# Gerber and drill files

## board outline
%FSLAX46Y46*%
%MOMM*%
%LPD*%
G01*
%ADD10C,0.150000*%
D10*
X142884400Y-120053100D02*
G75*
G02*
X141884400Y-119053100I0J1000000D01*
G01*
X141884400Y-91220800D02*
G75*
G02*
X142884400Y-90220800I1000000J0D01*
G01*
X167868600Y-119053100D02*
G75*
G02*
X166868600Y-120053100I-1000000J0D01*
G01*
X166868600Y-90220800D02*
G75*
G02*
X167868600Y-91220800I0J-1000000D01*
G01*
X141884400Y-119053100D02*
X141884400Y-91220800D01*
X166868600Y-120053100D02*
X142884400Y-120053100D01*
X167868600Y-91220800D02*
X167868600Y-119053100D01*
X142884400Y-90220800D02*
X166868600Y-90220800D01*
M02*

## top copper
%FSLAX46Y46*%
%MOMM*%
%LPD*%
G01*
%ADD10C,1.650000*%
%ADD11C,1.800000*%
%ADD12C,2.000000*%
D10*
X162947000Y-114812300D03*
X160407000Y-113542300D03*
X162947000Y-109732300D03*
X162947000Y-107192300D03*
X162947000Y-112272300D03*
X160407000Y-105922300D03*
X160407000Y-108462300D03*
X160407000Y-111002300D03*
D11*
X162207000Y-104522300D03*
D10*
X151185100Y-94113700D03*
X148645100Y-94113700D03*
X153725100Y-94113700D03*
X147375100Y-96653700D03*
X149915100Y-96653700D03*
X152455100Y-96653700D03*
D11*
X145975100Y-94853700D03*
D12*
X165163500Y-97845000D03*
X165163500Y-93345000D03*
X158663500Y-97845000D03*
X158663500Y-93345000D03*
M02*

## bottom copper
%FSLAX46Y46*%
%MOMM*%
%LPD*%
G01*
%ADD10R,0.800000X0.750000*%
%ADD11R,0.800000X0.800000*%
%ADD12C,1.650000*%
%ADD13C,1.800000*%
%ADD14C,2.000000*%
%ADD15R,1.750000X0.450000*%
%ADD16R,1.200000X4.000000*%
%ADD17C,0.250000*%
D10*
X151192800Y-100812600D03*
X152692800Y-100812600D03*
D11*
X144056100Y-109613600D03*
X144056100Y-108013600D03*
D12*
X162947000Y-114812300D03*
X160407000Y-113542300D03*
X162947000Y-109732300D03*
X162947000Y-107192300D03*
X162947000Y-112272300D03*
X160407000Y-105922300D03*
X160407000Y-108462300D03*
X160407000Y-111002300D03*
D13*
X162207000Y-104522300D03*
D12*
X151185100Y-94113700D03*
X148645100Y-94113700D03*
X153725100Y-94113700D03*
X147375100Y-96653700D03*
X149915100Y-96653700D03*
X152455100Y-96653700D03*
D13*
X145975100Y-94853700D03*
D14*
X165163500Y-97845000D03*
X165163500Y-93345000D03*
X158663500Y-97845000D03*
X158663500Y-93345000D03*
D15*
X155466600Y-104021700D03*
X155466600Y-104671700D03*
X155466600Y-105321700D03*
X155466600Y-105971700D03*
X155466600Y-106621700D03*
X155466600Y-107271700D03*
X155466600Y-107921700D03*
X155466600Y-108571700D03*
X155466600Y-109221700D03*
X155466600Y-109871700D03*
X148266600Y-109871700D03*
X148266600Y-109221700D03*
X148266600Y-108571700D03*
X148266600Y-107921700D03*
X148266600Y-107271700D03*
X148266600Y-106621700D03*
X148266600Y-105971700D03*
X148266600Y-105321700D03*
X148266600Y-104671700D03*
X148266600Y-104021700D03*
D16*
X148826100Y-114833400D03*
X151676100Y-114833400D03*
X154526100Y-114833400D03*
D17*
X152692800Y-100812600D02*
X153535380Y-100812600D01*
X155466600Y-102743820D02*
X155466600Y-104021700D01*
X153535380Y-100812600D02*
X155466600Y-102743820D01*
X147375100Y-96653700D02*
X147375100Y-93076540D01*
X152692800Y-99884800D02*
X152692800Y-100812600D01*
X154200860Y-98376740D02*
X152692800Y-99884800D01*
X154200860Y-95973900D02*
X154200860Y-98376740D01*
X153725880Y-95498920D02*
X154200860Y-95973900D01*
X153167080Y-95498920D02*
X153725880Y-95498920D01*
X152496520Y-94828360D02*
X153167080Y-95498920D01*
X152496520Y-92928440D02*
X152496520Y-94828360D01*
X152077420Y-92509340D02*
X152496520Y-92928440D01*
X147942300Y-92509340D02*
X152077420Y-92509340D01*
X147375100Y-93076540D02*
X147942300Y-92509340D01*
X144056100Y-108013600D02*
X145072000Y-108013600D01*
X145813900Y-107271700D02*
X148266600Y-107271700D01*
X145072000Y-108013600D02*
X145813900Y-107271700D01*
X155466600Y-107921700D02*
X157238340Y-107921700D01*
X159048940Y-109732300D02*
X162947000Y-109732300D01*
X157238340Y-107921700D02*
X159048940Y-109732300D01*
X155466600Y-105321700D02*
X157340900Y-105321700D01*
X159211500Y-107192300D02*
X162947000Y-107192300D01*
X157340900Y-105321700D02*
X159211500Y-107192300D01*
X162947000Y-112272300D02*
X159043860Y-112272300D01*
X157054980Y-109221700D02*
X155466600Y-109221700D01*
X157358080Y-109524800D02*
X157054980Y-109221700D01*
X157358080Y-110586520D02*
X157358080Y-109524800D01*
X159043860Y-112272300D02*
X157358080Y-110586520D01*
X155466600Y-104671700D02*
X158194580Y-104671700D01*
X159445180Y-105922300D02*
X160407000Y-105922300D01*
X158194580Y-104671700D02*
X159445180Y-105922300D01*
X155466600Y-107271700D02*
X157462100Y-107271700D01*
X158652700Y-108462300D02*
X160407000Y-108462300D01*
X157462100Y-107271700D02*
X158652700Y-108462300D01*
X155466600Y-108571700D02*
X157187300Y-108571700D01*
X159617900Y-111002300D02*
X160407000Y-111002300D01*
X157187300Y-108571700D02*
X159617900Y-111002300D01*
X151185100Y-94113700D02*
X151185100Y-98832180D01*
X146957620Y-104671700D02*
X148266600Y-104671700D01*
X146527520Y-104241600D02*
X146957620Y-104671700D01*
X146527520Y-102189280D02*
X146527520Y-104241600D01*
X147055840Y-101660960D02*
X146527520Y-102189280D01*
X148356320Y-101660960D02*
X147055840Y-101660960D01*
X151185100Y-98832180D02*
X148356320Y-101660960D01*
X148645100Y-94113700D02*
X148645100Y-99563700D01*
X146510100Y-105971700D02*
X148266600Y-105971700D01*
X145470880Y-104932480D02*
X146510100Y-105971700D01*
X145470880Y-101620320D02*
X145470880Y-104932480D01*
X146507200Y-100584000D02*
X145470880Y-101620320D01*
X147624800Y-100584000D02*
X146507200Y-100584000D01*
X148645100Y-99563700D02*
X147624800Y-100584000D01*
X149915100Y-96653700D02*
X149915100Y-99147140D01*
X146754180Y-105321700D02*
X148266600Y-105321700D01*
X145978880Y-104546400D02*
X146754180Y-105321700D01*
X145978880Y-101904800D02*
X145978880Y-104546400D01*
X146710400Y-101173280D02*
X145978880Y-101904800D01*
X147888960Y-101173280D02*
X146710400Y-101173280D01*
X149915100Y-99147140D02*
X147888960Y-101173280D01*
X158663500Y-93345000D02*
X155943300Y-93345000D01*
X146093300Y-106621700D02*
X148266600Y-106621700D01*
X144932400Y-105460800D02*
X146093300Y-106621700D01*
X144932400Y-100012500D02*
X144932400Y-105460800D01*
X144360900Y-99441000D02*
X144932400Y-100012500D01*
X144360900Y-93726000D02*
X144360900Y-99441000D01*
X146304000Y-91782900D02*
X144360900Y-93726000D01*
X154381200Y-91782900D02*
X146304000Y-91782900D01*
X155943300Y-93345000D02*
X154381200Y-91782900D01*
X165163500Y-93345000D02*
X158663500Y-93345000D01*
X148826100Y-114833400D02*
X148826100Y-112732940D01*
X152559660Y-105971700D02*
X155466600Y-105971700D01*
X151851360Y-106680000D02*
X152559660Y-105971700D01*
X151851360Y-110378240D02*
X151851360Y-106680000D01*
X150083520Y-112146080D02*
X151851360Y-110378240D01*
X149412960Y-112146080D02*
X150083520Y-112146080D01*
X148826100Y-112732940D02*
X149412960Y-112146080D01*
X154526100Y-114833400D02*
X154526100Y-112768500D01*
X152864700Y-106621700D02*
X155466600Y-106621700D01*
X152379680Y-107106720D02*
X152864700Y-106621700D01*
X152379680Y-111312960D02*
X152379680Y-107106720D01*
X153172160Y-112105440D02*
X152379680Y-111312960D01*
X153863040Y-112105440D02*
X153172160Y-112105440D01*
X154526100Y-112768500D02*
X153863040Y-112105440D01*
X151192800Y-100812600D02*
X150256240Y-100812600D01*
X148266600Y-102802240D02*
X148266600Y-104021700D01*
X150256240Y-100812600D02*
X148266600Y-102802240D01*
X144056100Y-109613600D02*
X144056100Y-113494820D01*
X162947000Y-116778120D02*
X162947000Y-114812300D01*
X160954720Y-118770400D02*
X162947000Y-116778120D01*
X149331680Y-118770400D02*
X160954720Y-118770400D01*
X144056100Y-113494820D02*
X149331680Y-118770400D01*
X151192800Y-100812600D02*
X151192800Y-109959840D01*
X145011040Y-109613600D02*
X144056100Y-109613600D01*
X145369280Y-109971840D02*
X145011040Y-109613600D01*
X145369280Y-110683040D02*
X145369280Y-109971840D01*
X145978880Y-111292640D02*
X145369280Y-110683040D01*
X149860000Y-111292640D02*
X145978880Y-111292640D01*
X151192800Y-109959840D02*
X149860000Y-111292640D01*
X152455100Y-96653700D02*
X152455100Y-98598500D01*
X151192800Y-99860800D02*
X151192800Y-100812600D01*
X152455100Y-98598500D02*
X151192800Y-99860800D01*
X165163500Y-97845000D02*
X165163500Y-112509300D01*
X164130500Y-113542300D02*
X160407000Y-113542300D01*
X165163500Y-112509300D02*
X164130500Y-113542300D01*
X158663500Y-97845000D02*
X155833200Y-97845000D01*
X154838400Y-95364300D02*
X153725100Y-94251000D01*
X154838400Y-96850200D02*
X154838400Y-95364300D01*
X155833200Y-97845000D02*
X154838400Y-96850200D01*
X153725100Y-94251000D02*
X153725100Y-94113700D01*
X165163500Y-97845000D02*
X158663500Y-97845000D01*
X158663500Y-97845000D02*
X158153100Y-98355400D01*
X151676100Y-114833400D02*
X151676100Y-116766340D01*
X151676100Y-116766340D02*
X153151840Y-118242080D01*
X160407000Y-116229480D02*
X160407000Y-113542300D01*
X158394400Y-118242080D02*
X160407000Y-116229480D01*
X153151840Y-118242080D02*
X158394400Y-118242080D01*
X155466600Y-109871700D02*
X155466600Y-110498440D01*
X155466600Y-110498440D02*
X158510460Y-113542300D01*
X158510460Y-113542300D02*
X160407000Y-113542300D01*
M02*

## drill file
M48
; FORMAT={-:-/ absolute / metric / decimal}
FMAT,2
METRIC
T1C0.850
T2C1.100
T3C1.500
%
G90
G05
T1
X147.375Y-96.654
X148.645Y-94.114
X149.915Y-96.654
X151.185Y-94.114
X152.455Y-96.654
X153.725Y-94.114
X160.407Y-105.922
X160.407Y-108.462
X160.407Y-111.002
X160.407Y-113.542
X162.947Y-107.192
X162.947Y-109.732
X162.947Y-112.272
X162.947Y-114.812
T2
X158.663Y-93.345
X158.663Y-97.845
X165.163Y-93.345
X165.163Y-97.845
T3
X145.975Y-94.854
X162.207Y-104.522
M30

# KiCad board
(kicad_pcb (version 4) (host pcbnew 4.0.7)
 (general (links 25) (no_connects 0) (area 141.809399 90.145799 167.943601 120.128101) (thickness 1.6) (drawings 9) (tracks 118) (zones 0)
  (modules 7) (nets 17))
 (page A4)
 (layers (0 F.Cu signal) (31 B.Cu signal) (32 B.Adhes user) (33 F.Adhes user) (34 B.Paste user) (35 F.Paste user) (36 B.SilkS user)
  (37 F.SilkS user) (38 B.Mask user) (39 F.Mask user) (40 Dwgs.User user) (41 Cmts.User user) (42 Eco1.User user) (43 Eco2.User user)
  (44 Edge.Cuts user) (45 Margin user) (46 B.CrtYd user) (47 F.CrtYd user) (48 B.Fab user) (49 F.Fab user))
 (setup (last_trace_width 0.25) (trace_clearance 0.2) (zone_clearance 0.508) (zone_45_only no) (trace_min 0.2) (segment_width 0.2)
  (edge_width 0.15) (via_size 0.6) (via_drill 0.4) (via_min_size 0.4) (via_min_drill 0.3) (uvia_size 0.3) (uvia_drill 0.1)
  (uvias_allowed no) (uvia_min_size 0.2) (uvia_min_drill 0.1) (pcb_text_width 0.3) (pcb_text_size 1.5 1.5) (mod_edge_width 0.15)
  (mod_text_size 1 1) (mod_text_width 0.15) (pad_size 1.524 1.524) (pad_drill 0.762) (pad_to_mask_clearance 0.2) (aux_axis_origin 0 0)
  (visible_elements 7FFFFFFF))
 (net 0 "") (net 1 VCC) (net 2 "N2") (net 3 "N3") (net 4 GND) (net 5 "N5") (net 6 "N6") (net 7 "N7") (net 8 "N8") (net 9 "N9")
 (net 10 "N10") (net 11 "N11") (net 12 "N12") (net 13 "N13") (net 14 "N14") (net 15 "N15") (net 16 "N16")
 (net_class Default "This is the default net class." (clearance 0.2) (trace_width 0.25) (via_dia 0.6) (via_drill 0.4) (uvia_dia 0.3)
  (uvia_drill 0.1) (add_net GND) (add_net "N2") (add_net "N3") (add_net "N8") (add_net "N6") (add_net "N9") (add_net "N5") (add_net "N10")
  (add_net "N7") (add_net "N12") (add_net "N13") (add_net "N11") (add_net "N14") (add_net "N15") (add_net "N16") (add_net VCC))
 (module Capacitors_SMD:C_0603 (layer B.Cu) (at 151.9428 100.8126 180)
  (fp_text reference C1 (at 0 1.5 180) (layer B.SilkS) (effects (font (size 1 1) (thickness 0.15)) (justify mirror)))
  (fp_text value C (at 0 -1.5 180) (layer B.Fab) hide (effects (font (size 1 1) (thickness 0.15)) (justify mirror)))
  (pad 2 smd rect (at 0.75 0 180) (size 0.8 0.75) (layers B.Cu B.Paste B.Mask) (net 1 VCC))
  (pad 1 smd rect (at -0.75 0 180) (size 0.8 0.75) (layers B.Cu B.Paste B.Mask) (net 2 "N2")))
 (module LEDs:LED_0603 (layer B.Cu) (at 144.0561 108.8136 270)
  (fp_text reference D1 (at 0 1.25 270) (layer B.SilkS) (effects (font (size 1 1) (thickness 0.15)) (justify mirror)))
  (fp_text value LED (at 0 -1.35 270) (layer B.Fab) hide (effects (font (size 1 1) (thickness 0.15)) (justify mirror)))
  (pad 2 smd rect (at 0.8 0 90) (size 0.8 0.8) (layers B.Cu B.Paste B.Mask) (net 1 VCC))
  (pad 1 smd rect (at -0.8 0 90) (size 0.8 0.8) (layers B.Cu B.Paste B.Mask) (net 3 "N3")))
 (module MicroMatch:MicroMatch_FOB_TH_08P (layer F.Cu) (at 166.497 106.0323 90)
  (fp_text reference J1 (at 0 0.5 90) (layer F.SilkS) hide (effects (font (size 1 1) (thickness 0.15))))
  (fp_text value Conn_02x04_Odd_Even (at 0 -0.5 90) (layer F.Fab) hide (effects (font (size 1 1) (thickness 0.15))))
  (pad 8 thru_hole circle (at -8.78 -3.55 90) (size 1.65 1.65) (drill 0.85) (layers *.Cu *.Mask) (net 1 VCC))
  (pad 7 thru_hole circle (at -7.51 -6.09 90) (size 1.65 1.65) (drill 0.85) (layers *.Cu *.Mask) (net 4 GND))
  (pad 4 thru_hole circle (at -3.7 -3.55 90) (size 1.65 1.65) (drill 0.85) (layers *.Cu *.Mask) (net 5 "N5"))
  (pad 2 thru_hole circle (at -1.16 -3.55 90) (size 1.65 1.65) (drill 0.85) (layers *.Cu *.Mask) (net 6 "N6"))
  (pad 6 thru_hole circle (at -6.24 -3.55 90) (size 1.65 1.65) (drill 0.85) (layers *.Cu *.Mask) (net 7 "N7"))
  (pad 1 thru_hole circle (at 0.11 -6.09 90) (size 1.65 1.65) (drill 0.85) (layers *.Cu *.Mask) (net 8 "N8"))
  (pad 3 thru_hole circle (at -2.43 -6.09 90) (size 1.65 1.65) (drill 0.85) (layers *.Cu *.Mask) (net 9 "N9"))
  (pad 5 thru_hole circle (at -4.97 -6.09 90) (size 1.65 1.65) (drill 0.85) (layers *.Cu *.Mask) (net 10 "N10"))
  (pad "" np_thru_hole circle (at 1.51 -4.29 90) (size 1.8 1.8) (drill 1.5) (layers *.Cu *.Mask)))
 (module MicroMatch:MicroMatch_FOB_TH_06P (layer F.Cu) (at 147.4851 90.5637 180)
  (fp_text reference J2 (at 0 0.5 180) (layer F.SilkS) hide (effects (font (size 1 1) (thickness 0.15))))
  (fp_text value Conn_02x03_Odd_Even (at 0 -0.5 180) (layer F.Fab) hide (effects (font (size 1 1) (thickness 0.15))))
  (pad 4 thru_hole circle (at -3.7 -3.55 180) (size 1.65 1.65) (drill 0.85) (layers *.Cu *.Mask) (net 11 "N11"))
  (pad 2 thru_hole circle (at -1.16 -3.55 180) (size 1.65 1.65) (drill 0.85) (layers *.Cu *.Mask) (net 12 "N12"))
  (pad 6 thru_hole circle (at -6.24 -3.55 180) (size 1.65 1.65) (drill 0.85) (layers *.Cu *.Mask) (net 4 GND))
  (pad 1 thru_hole circle (at 0.11 -6.09 180) (size 1.65 1.65) (drill 0.85) (layers *.Cu *.Mask) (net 2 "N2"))
  (pad 3 thru_hole circle (at -2.43 -6.09 180) (size 1.65 1.65) (drill 0.85) (layers *.Cu *.Mask) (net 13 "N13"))
  (pad 5 thru_hole circle (at -4.97 -6.09 180) (size 1.65 1.65) (drill 0.85) (layers *.Cu *.Mask) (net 1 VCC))
  (pad "" np_thru_hole circle (at 1.51 -4.29 180) (size 1.8 1.8) (drill 1.5) (layers *.Cu *.Mask)))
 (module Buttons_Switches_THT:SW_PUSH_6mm (layer B.Cu) (at 165.1635 93.345 180)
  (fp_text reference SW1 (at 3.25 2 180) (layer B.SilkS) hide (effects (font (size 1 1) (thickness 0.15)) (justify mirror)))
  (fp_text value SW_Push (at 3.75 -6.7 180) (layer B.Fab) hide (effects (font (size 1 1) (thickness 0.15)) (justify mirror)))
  (pad 2 thru_hole circle (at 0 -4.5 90) (size 2 2) (drill 1.1) (layers *.Cu *.Mask) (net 4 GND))
  (pad 1 thru_hole circle (at 0 0 90) (size 2 2) (drill 1.1) (layers *.Cu *.Mask) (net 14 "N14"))
  (pad 2 thru_hole circle (at 6.5 -4.5 90) (size 2 2) (drill 1.1) (layers *.Cu *.Mask) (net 4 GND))
  (pad 1 thru_hole circle (at 6.5 0 90) (size 2 2) (drill 1.1) (layers *.Cu *.Mask) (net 14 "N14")))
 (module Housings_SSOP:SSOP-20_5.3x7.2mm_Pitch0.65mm (layer B.Cu) (at 151.8666 106.9467 180)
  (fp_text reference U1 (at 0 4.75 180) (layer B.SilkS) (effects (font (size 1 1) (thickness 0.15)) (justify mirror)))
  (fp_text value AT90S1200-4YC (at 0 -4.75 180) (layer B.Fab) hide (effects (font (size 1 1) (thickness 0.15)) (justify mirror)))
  (pad 1 smd rect (at -3.6 2.925 180) (size 1.75 0.45) (layers B.Cu B.Paste B.Mask) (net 2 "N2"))
  (pad 2 smd rect (at -3.6 2.275 180) (size 1.75 0.45) (layers B.Cu B.Paste B.Mask) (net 8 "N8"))
  (pad 3 smd rect (at -3.6 1.625 180) (size 1.75 0.45) (layers B.Cu B.Paste B.Mask) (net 6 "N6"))
  (pad 4 smd rect (at -3.6 0.975 180) (size 1.75 0.45) (layers B.Cu B.Paste B.Mask) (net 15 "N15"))
  (pad 5 smd rect (at -3.6 0.325 180) (size 1.75 0.45) (layers B.Cu B.Paste B.Mask) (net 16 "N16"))
  (pad 6 smd rect (at -3.6 -0.325 180) (size 1.75 0.45) (layers B.Cu B.Paste B.Mask) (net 9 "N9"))
  (pad 7 smd rect (at -3.6 -0.975 180) (size 1.75 0.45) (layers B.Cu B.Paste B.Mask) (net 5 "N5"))
  (pad 8 smd rect (at -3.6 -1.625 180) (size 1.75 0.45) (layers B.Cu B.Paste B.Mask) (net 10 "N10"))
  (pad 9 smd rect (at -3.6 -2.275 180) (size 1.75 0.45) (layers B.Cu B.Paste B.Mask) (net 7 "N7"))
  (pad 10 smd rect (at -3.6 -2.925 180) (size 1.75 0.45) (layers B.Cu B.Paste B.Mask) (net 4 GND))
  (pad 11 smd rect (at 3.6 -2.925 180) (size 1.75 0.45) (layers B.Cu B.Paste B.Mask))
  (pad 12 smd rect (at 3.6 -2.275 180) (size 1.75 0.45) (layers B.Cu B.Paste B.Mask))
  (pad 13 smd rect (at 3.6 -1.625 180) (size 1.75 0.45) (layers B.Cu B.Paste B.Mask))
  (pad 14 smd rect (at 3.6 -0.975 180) (size 1.75 0.45) (layers B.Cu B.Paste B.Mask))
  (pad 15 smd rect (at 3.6 -0.325 180) (size 1.75 0.45) (layers B.Cu B.Paste B.Mask) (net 3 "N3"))
  (pad 16 smd rect (at 3.6 0.325 180) (size 1.75 0.45) (layers B.Cu B.Paste B.Mask) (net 14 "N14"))
  (pad 17 smd rect (at 3.6 0.975 180) (size 1.75 0.45) (layers B.Cu B.Paste B.Mask) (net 12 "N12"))
  (pad 18 smd rect (at 3.6 1.625 180) (size 1.75 0.45) (layers B.Cu B.Paste B.Mask) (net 13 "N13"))
  (pad 19 smd rect (at 3.6 2.275 180) (size 1.75 0.45) (layers B.Cu B.Paste B.Mask) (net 11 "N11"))
  (pad 20 smd rect (at 3.6 2.925 180) (size 1.75 0.45) (layers B.Cu B.Paste B.Mask) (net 1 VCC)))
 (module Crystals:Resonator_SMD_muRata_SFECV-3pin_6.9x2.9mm (layer B.Cu) (at 151.6761 114.8334)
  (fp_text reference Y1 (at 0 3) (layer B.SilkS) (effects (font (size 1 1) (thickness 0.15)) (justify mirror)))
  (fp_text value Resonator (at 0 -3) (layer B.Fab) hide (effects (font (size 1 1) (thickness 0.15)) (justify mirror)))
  (pad 1 smd rect (at -2.85 0) (size 1.2 4) (layers B.Cu B.Paste B.Mask) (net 15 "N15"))
  (pad 2 smd rect (at 0 0) (size 1.2 4) (layers B.Cu B.Paste B.Mask) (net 4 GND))
  (pad 3 smd rect (at 2.85 0) (size 1.2 4) (layers B.Cu B.Paste B.Mask) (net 16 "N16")))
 (gr_arc (start 142.8844 119.0531) (end 142.8844 120.0531) (angle 90) (layer Edge.Cuts) (width 0.15))
 (gr_arc (start 142.8844 91.2208) (end 141.8844 91.2208) (angle 90) (layer Edge.Cuts) (width 0.15))
 (gr_arc (start 166.8686 119.0531) (end 167.8686 119.0531) (angle 90) (layer Edge.Cuts) (width 0.15))
 (gr_arc (start 166.8686 91.2208) (end 166.8686 90.2208) (angle 90) (layer Edge.Cuts) (width 0.15))
 (gr_line (start 141.8844 119.0531) (end 141.8844 91.2208) (angle 90) (layer Edge.Cuts) (width 0.15))
 (gr_line (start 166.8686 120.0531) (end 142.8844 120.0531) (angle 90) (layer Edge.Cuts) (width 0.15))
 (gr_line (start 167.8686 91.2208) (end 167.8686 119.0531) (angle 90) (layer Edge.Cuts) (width 0.15))
 (gr_line (start 142.8844 90.2208) (end 166.8686 90.2208) (angle 90) (layer Edge.Cuts) (width 0.15))
 (segment (start 152.6928 100.8126) (end 153.53538 100.8126) (width 0.25) (layer B.Cu) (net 2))
 (segment (start 155.4666 102.74382) (end 155.4666 104.0217) (width 0.25) (layer B.Cu) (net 2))
 (segment (start 153.53538 100.8126) (end 155.4666 102.74382) (width 0.25) (layer B.Cu) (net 2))
 (segment (start 147.3751 96.6537) (end 147.3751 93.07654) (width 0.25) (layer B.Cu) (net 2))
 (segment (start 152.6928 99.8848) (end 152.6928 100.8126) (width 0.25) (layer B.Cu) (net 2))
 (segment (start 154.20086 98.37674) (end 152.6928 99.8848) (width 0.25) (layer B.Cu) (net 2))
 (segment (start 154.20086 95.9739) (end 154.20086 98.37674) (width 0.25) (layer B.Cu) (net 2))
 (segment (start 153.72588 95.49892) (end 154.20086 95.9739) (width 0.25) (layer B.Cu) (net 2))
 (segment (start 153.16708 95.49892) (end 153.72588 95.49892) (width 0.25) (layer B.Cu) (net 2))
 (segment (start 152.49652 94.82836) (end 153.16708 95.49892) (width 0.25) (layer B.Cu) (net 2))
 (segment (start 152.49652 92.92844) (end 152.49652 94.82836) (width 0.25) (layer B.Cu) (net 2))
 (segment (start 152.07742 92.50934) (end 152.49652 92.92844) (width 0.25) (layer B.Cu) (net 2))
 (segment (start 147.9423 92.50934) (end 152.07742 92.50934) (width 0.25) (layer B.Cu) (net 2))
 (segment (start 147.3751 93.07654) (end 147.9423 92.50934) (width 0.25) (layer B.Cu) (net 2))
 (segment (start 144.0561 108.0136) (end 145.072 108.0136) (width 0.25) (layer B.Cu) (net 3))
 (segment (start 145.8139 107.2717) (end 148.2666 107.2717) (width 0.25) (layer B.Cu) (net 3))
 (segment (start 145.072 108.0136) (end 145.8139 107.2717) (width 0.25) (layer B.Cu) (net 3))
 (segment (start 155.4666 107.9217) (end 157.23834 107.9217) (width 0.25) (layer B.Cu) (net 5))
 (segment (start 159.04894 109.7323) (end 162.947 109.7323) (width 0.25) (layer B.Cu) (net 5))
 (segment (start 157.23834 107.9217) (end 159.04894 109.7323) (width 0.25) (layer B.Cu) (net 5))
 (segment (start 155.4666 105.3217) (end 157.3409 105.3217) (width 0.25) (layer B.Cu) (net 6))
 (segment (start 159.2115 107.1923) (end 162.947 107.1923) (width 0.25) (layer B.Cu) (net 6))
 (segment (start 157.3409 105.3217) (end 159.2115 107.1923) (width 0.25) (layer B.Cu) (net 6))
 (segment (start 162.947 112.2723) (end 159.04386 112.2723) (width 0.25) (layer B.Cu) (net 7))
 (segment (start 157.05498 109.2217) (end 155.4666 109.2217) (width 0.25) (layer B.Cu) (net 7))
 (segment (start 157.35808 109.5248) (end 157.05498 109.2217) (width 0.25) (layer B.Cu) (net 7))
 (segment (start 157.35808 110.58652) (end 157.35808 109.5248) (width 0.25) (layer B.Cu) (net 7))
 (segment (start 159.04386 112.2723) (end 157.35808 110.58652) (width 0.25) (layer B.Cu) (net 7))
 (segment (start 155.4666 104.6717) (end 158.19458 104.6717) (width 0.25) (layer B.Cu) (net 8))
 (segment (start 159.44518 105.9223) (end 160.407 105.9223) (width 0.25) (layer B.Cu) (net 8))
 (segment (start 158.19458 104.6717) (end 159.44518 105.9223) (width 0.25) (layer B.Cu) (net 8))
 (segment (start 155.4666 107.2717) (end 157.4621 107.2717) (width 0.25) (layer B.Cu) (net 9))
 (segment (start 158.6527 108.4623) (end 160.407 108.4623) (width 0.25) (layer B.Cu) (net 9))
 (segment (start 157.4621 107.2717) (end 158.6527 108.4623) (width 0.25) (layer B.Cu) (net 9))
 (segment (start 155.4666 108.5717) (end 157.1873 108.5717) (width 0.25) (layer B.Cu) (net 10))
 (segment (start 159.6179 111.0023) (end 160.407 111.0023) (width 0.25) (layer B.Cu) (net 10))
 (segment (start 157.1873 108.5717) (end 159.6179 111.0023) (width 0.25) (layer B.Cu) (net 10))
 (segment (start 151.1851 94.1137) (end 151.1851 98.83218) (width 0.25) (layer B.Cu) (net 11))
 (segment (start 146.95762 104.6717) (end 148.2666 104.6717) (width 0.25) (layer B.Cu) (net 11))
 (segment (start 146.52752 104.2416) (end 146.95762 104.6717) (width 0.25) (layer B.Cu) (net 11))
 (segment (start 146.52752 102.18928) (end 146.52752 104.2416) (width 0.25) (layer B.Cu) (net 11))
 (segment (start 147.05584 101.66096) (end 146.52752 102.18928) (width 0.25) (layer B.Cu) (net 11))
 (segment (start 148.35632 101.66096) (end 147.05584 101.66096) (width 0.25) (layer B.Cu) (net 11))
 (segment (start 151.1851 98.83218) (end 148.35632 101.66096) (width 0.25) (layer B.Cu) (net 11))
 (segment (start 148.6451 94.1137) (end 148.6451 99.5637) (width 0.25) (layer B.Cu) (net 12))
 (segment (start 146.5101 105.9717) (end 148.2666 105.9717) (width 0.25) (layer B.Cu) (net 12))
 (segment (start 145.47088 104.93248) (end 146.5101 105.9717) (width 0.25) (layer B.Cu) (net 12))
 (segment (start 145.47088 101.62032) (end 145.47088 104.93248) (width 0.25) (layer B.Cu) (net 12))
 (segment (start 146.5072 100.584) (end 145.47088 101.62032) (width 0.25) (layer B.Cu) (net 12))
 (segment (start 147.6248 100.584) (end 146.5072 100.584) (width 0.25) (layer B.Cu) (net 12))
 (segment (start 148.6451 99.5637) (end 147.6248 100.584) (width 0.25) (layer B.Cu) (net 12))
 (segment (start 149.9151 96.6537) (end 149.9151 99.14714) (width 0.25) (layer B.Cu) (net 13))
 (segment (start 146.75418 105.3217) (end 148.2666 105.3217) (width 0.25) (layer B.Cu) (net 13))
 (segment (start 145.97888 104.5464) (end 146.75418 105.3217) (width 0.25) (layer B.Cu) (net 13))
 (segment (start 145.97888 101.9048) (end 145.97888 104.5464) (width 0.25) (layer B.Cu) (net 13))
 (segment (start 146.7104 101.17328) (end 145.97888 101.9048) (width 0.25) (layer B.Cu) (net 13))
 (segment (start 147.88896 101.17328) (end 146.7104 101.17328) (width 0.25) (layer B.Cu) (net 13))
 (segment (start 149.9151 99.14714) (end 147.88896 101.17328) (width 0.25) (layer B.Cu) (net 13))
 (segment (start 158.6635 93.345) (end 155.9433 93.345) (width 0.25) (layer B.Cu) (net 14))
 (segment (start 146.0933 106.6217) (end 148.2666 106.6217) (width 0.25) (layer B.Cu) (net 14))
 (segment (start 144.9324 105.4608) (end 146.0933 106.6217) (width 0.25) (layer B.Cu) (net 14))
 (segment (start 144.9324 100.0125) (end 144.9324 105.4608) (width 0.25) (layer B.Cu) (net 14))
 (segment (start 144.3609 99.441) (end 144.9324 100.0125) (width 0.25) (layer B.Cu) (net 14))
 (segment (start 144.3609 93.726) (end 144.3609 99.441) (width 0.25) (layer B.Cu) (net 14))
 (segment (start 146.304 91.7829) (end 144.3609 93.726) (width 0.25) (layer B.Cu) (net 14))
 (segment (start 154.3812 91.7829) (end 146.304 91.7829) (width 0.25) (layer B.Cu) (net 14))
 (segment (start 155.9433 93.345) (end 154.3812 91.7829) (width 0.25) (layer B.Cu) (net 14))
 (segment (start 165.1635 93.345) (end 158.6635 93.345) (width 0.25) (layer B.Cu) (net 14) (status 30))
 (segment (start 148.8261 114.8334) (end 148.8261 112.73294) (width 0.25) (layer B.Cu) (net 15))
 (segment (start 152.55966 105.9717) (end 155.4666 105.9717) (width 0.25) (layer B.Cu) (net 15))
 (segment (start 151.85136 106.68) (end 152.55966 105.9717) (width 0.25) (layer B.Cu) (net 15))
 (segment (start 151.85136 110.37824) (end 151.85136 106.68) (width 0.25) (layer B.Cu) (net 15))
 (segment (start 150.08352 112.14608) (end 151.85136 110.37824) (width 0.25) (layer B.Cu) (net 15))
 (segment (start 149.41296 112.14608) (end 150.08352 112.14608) (width 0.25) (layer B.Cu) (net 15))
 (segment (start 148.8261 112.73294) (end 149.41296 112.14608) (width 0.25) (layer B.Cu) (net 15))
 (segment (start 154.5261 114.8334) (end 154.5261 112.7685) (width 0.25) (layer B.Cu) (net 16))
 (segment (start 152.8647 106.6217) (end 155.4666 106.6217) (width 0.25) (layer B.Cu) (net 16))
 (segment (start 152.37968 107.10672) (end 152.8647 106.6217) (width 0.25) (layer B.Cu) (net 16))
 (segment (start 152.37968 111.31296) (end 152.37968 107.10672) (width 0.25) (layer B.Cu) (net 16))
 (segment (start 153.17216 112.10544) (end 152.37968 111.31296) (width 0.25) (layer B.Cu) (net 16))
 (segment (start 153.86304 112.10544) (end 153.17216 112.10544) (width 0.25) (layer B.Cu) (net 16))
 (segment (start 154.5261 112.7685) (end 153.86304 112.10544) (width 0.25) (layer B.Cu) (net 16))
 (segment (start 151.1928 100.8126) (end 150.25624 100.8126) (width 0.25) (layer B.Cu) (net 1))
 (segment (start 148.2666 102.80224) (end 148.2666 104.0217) (width 0.25) (layer B.Cu) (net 1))
 (segment (start 150.25624 100.8126) (end 148.2666 102.80224) (width 0.25) (layer B.Cu) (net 1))
 (segment (start 144.0561 109.6136) (end 144.0561 113.49482) (width 0.25) (layer B.Cu) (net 1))
 (segment (start 162.947 116.77812) (end 162.947 114.8123) (width 0.25) (layer B.Cu) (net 1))
 (segment (start 160.95472 118.7704) (end 162.947 116.77812) (width 0.25) (layer B.Cu) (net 1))
 (segment (start 149.33168 118.7704) (end 160.95472 118.7704) (width 0.25) (layer B.Cu) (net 1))
 (segment (start 144.0561 113.49482) (end 149.33168 118.7704) (width 0.25) (layer B.Cu) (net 1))
 (segment (start 151.1928 100.8126) (end 151.1928 109.95984) (width 0.25) (layer B.Cu) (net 1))
 (segment (start 145.01104 109.6136) (end 144.0561 109.6136) (width 0.25) (layer B.Cu) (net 1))
 (segment (start 145.36928 109.97184) (end 145.01104 109.6136) (width 0.25) (layer B.Cu) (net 1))
 (segment (start 145.36928 110.68304) (end 145.36928 109.97184) (width 0.25) (layer B.Cu) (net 1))
 (segment (start 145.97888 111.29264) (end 145.36928 110.68304) (width 0.25) (layer B.Cu) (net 1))
 (segment (start 149.86 111.29264) (end 145.97888 111.29264) (width 0.25) (layer B.Cu) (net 1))
 (segment (start 151.1928 109.95984) (end 149.86 111.29264) (width 0.25) (layer B.Cu) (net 1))
 (segment (start 152.4551 96.6537) (end 152.4551 98.5985) (width 0.25) (layer B.Cu) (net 1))
 (segment (start 151.1928 99.8608) (end 151.1928 100.8126) (width 0.25) (layer B.Cu) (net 1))
 (segment (start 152.4551 98.5985) (end 151.1928 99.8608) (width 0.25) (layer B.Cu) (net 1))
 (segment (start 165.1635 97.845) (end 165.1635 112.5093) (width 0.25) (layer B.Cu) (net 4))
 (segment (start 164.1305 113.5423) (end 160.407 113.5423) (width 0.25) (layer B.Cu) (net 4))
 (segment (start 165.1635 112.5093) (end 164.1305 113.5423) (width 0.25) (layer B.Cu) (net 4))
 (segment (start 158.6635 97.845) (end 155.8332 97.845) (width 0.25) (layer B.Cu) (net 4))
 (segment (start 154.8384 95.3643) (end 153.7251 94.251) (width 0.25) (layer B.Cu) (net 4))
 (segment (start 154.8384 96.8502) (end 154.8384 95.3643) (width 0.25) (layer B.Cu) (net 4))
 (segment (start 155.8332 97.845) (end 154.8384 96.8502) (width 0.25) (layer B.Cu) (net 4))
 (segment (start 153.7251 94.251) (end 153.7251 94.1137) (width 0.25) (layer B.Cu) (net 4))
 (segment (start 165.1635 97.845) (end 158.6635 97.845) (width 0.25) (layer B.Cu) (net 4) (status 30))
 (segment (start 158.6635 97.845) (end 158.1531 98.3554) (width 0.25) (layer B.Cu) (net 4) (status 30))
 (segment (start 151.6761 114.8334) (end 151.6761 116.76634) (width 0.25) (layer B.Cu) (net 4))
 (segment (start 151.6761 116.76634) (end 153.15184 118.24208) (width 0.25) (layer B.Cu) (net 4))
 (segment (start 160.407 116.22948) (end 160.407 113.5423) (width 0.25) (layer B.Cu) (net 4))
 (segment (start 158.3944 118.24208) (end 160.407 116.22948) (width 0.25) (layer B.Cu) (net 4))
 (segment (start 153.15184 118.24208) (end 158.3944 118.24208) (width 0.25) (layer B.Cu) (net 4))
 (segment (start 155.4666 109.8717) (end 155.4666 110.49844) (width 0.25) (layer B.Cu) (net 4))
 (segment (start 155.4666 110.49844) (end 158.51046 113.5423) (width 0.25) (layer B.Cu) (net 4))
 (segment (start 158.51046 113.5423) (end 160.407 113.5423) (width 0.25) (layer B.Cu) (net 4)))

